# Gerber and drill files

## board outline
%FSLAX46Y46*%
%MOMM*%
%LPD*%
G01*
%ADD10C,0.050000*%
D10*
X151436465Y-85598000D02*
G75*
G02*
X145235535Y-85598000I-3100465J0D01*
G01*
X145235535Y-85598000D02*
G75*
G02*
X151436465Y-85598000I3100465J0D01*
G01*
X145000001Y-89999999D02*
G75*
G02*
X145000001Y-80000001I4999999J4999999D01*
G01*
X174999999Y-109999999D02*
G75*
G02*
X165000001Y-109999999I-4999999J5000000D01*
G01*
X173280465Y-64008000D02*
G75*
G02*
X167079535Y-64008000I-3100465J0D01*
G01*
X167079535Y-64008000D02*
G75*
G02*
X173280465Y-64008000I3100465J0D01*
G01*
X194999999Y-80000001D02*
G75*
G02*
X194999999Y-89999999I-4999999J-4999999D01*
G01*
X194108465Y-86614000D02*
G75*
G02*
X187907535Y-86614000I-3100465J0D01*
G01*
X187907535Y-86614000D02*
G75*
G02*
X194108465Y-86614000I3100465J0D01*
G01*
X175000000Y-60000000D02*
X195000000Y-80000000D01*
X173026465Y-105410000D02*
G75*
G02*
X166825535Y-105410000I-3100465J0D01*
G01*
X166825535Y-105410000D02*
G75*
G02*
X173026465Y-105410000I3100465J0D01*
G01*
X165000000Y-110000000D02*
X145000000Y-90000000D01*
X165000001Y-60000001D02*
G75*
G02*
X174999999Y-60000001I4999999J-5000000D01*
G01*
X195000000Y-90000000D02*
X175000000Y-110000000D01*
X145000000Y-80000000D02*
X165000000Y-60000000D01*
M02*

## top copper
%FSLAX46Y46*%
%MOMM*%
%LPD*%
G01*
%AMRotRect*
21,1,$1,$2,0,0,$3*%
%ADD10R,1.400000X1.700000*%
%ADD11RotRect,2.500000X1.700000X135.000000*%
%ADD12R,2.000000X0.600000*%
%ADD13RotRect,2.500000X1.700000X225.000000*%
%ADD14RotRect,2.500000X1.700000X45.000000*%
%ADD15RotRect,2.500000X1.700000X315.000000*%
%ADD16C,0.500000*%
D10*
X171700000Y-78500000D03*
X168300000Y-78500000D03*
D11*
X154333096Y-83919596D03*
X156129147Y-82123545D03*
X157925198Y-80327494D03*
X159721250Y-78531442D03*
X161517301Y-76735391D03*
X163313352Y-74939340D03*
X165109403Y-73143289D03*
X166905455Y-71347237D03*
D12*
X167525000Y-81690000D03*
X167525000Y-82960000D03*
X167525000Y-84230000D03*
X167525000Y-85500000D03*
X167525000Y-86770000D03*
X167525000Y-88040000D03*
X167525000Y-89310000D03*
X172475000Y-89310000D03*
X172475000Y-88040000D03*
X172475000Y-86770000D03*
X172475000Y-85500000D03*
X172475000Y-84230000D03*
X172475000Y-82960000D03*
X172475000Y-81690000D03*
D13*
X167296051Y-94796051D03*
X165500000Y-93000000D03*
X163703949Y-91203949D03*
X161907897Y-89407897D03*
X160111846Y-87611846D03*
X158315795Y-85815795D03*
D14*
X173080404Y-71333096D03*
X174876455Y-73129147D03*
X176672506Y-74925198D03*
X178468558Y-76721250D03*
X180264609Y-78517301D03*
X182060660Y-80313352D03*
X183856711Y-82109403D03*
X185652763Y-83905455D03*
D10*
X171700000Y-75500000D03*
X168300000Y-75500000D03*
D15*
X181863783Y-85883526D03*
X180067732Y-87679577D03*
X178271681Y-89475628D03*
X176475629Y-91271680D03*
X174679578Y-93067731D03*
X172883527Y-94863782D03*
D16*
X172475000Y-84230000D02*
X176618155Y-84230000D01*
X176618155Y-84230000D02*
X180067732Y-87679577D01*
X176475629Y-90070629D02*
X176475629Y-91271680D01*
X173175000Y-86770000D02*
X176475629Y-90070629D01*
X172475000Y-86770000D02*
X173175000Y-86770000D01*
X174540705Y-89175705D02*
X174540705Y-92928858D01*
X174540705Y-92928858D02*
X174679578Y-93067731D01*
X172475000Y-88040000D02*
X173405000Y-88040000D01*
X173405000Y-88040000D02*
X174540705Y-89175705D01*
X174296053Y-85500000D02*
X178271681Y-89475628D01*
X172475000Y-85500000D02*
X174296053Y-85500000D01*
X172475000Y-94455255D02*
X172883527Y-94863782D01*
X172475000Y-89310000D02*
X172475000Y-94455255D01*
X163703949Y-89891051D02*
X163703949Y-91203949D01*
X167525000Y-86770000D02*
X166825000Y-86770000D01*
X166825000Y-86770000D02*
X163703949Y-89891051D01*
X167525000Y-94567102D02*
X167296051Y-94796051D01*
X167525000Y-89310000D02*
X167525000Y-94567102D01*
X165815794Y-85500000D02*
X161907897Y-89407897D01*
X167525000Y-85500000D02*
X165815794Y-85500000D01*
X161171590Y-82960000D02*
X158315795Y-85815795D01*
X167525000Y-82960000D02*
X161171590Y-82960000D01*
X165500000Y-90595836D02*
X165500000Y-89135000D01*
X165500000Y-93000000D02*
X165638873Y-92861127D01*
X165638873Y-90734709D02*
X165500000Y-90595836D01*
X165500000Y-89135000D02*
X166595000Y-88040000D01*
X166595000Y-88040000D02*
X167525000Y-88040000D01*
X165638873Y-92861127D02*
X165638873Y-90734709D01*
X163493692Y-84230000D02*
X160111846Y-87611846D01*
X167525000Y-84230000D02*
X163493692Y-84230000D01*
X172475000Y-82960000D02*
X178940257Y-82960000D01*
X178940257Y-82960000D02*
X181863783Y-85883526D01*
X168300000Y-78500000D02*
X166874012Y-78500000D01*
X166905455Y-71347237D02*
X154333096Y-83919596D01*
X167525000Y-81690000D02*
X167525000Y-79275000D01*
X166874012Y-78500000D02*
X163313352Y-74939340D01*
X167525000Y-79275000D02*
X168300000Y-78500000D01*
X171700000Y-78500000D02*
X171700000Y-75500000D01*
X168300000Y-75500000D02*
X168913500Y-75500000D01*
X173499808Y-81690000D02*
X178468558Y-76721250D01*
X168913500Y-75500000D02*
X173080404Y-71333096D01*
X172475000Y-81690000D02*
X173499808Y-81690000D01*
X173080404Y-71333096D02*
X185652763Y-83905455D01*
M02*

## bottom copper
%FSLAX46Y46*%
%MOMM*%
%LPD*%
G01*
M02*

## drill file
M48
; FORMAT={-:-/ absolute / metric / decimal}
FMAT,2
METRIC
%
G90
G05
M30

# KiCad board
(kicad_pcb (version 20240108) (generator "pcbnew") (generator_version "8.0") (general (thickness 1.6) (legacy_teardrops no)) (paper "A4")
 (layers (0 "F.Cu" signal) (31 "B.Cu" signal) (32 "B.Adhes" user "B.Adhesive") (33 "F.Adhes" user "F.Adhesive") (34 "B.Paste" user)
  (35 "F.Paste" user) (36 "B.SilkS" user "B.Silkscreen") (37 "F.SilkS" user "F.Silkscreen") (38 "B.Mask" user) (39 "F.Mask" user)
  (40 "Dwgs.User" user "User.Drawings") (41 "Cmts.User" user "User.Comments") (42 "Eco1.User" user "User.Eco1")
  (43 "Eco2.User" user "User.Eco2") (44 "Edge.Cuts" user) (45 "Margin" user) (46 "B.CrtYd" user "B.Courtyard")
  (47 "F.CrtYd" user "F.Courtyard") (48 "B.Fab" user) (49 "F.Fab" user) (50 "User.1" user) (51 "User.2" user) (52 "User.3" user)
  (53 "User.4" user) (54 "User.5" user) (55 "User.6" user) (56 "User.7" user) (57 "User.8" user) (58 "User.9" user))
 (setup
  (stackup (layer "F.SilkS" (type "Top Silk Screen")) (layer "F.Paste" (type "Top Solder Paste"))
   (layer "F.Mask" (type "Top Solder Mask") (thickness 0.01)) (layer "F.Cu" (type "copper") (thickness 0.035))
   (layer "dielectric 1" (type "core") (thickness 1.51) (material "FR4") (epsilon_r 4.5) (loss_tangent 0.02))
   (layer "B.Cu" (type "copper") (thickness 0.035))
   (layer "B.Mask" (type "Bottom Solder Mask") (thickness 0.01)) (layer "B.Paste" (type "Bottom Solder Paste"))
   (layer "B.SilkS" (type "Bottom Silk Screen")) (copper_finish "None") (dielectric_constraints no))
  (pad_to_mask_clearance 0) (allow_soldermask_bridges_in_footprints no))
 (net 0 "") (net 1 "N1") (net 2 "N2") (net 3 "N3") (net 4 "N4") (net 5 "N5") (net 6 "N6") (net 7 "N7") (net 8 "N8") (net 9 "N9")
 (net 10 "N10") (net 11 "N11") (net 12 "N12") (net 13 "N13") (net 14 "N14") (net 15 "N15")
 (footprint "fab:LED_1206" (layer "F.Cu") (at 170 78.5 180)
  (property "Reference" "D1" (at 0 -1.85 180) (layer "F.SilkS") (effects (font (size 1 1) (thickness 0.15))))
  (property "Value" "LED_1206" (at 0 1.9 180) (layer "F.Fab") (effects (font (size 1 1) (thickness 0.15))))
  (pad "1" smd rect (at -1.7 0 180) (size 1.4 1.7) (layers "F.Cu" "F.Paste" "F.Mask") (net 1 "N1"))
  (pad "2" smd rect (at 1.7 0 180) (size 1.4 1.7) (layers "F.Cu" "F.Paste" "F.Mask") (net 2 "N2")))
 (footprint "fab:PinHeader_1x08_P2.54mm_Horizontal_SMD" (layer "F.Cu") (at 154.333096 83.919596 135)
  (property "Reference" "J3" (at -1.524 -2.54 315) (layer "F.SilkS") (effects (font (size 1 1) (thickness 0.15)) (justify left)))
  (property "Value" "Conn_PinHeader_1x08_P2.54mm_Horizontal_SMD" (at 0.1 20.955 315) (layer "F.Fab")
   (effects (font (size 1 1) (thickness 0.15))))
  (pad "1" smd rect (at 0 0 135) (size 2.5 1.7) (layers "F.Cu" "F.Paste" "F.Mask") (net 2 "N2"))
  (pad "2" smd rect (at 0 2.54 135) (size 2.5 1.7) (layers "F.Cu" "F.Paste" "F.Mask") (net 2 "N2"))
  (pad "3" smd rect (at 0 5.079999 135) (size 2.5 1.7) (layers "F.Cu" "F.Paste" "F.Mask") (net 2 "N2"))
  (pad "4" smd rect (at 0 7.62 135) (size 2.5 1.7) (layers "F.Cu" "F.Paste" "F.Mask") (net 2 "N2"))
  (pad "5" smd rect (at 0 10.16 135) (size 2.5 1.7) (layers "F.Cu" "F.Paste" "F.Mask") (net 2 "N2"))
  (pad "6" smd rect (at 0 12.7 135) (size 2.5 1.7) (layers "F.Cu" "F.Paste" "F.Mask") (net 2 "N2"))
  (pad "7" smd rect (at 0 15.24 135) (size 2.5 1.7) (layers "F.Cu" "F.Paste" "F.Mask") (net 2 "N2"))
  (pad "8" smd rect (at 0 17.780001 135) (size 2.5 1.7) (layers "F.Cu" "F.Paste" "F.Mask") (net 2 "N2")))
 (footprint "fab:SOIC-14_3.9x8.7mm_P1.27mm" (layer "F.Cu") (at 170 85.5)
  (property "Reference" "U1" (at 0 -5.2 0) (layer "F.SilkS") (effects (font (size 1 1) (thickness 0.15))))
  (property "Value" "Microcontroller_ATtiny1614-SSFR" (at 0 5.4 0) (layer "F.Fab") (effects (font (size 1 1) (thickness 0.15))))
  (pad "1" smd rect (at -2.475 -3.81) (size 2 0.6) (layers "F.Cu" "F.Paste" "F.Mask") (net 2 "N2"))
  (pad "2" smd rect (at -2.475 -2.54) (size 2 0.6) (layers "F.Cu" "F.Paste" "F.Mask") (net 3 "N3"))
  (pad "3" smd rect (at -2.475 -1.27) (size 2 0.6) (layers "F.Cu" "F.Paste" "F.Mask") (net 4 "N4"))
  (pad "4" smd rect (at -2.475 0) (size 2 0.6) (layers "F.Cu" "F.Paste" "F.Mask") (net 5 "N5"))
  (pad "5" smd rect (at -2.475 1.27) (size 2 0.6) (layers "F.Cu" "F.Paste" "F.Mask") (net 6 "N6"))
  (pad "6" smd rect (at -2.475 2.54) (size 2 0.6) (layers "F.Cu" "F.Paste" "F.Mask") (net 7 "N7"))
  (pad "7" smd rect (at -2.475 3.81) (size 2 0.6) (layers "F.Cu" "F.Paste" "F.Mask") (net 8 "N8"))
  (pad "8" smd rect (at 2.475 3.81) (size 2 0.6) (layers "F.Cu" "F.Paste" "F.Mask") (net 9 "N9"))
  (pad "9" smd rect (at 2.475 2.54) (size 2 0.6) (layers "F.Cu" "F.Paste" "F.Mask") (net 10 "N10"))
  (pad "10" smd rect (at 2.475 1.27) (size 2 0.6) (layers "F.Cu" "F.Paste" "F.Mask") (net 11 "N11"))
  (pad "11" smd rect (at 2.475 0) (size 2 0.6) (layers "F.Cu" "F.Paste" "F.Mask") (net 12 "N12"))
  (pad "12" smd rect (at 2.475 -1.27) (size 2 0.6) (layers "F.Cu" "F.Paste" "F.Mask") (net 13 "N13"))
  (pad "13" smd rect (at 2.475 -2.54) (size 2 0.6) (layers "F.Cu" "F.Paste" "F.Mask") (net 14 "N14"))
  (pad "14" smd rect (at 2.475 -3.81) (size 2 0.6) (layers "F.Cu" "F.Paste" "F.Mask") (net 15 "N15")))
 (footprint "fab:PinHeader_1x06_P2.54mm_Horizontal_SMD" (layer "F.Cu") (at 167.296051 94.796051 -135)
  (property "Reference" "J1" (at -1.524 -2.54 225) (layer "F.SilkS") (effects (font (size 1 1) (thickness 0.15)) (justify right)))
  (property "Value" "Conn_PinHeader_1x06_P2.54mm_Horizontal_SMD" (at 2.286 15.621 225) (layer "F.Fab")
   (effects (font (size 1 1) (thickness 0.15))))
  (pad "1" smd rect (at 0 0 225) (size 2.5 1.7) (layers "F.Cu" "F.Paste" "F.Mask") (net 8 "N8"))
  (pad "2" smd rect (at 0 2.54 225) (size 2.5 1.7) (layers "F.Cu" "F.Paste" "F.Mask") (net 7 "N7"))
  (pad "3" smd rect (at 0 5.079999 225) (size 2.5 1.7) (layers "F.Cu" "F.Paste" "F.Mask") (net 6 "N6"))
  (pad "4" smd rect (at 0 7.62 225) (size 2.5 1.7) (layers "F.Cu" "F.Paste" "F.Mask") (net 5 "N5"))
  (pad "5" smd rect (at 0 10.16 225) (size 2.5 1.7) (layers "F.Cu" "F.Paste" "F.Mask") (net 4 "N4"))
  (pad "6" smd rect (at 0 12.7 225) (size 2.5 1.7) (layers "F.Cu" "F.Paste" "F.Mask") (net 3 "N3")))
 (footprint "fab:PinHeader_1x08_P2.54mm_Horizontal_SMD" (layer "F.Cu") (at 173.080404 71.333096 45)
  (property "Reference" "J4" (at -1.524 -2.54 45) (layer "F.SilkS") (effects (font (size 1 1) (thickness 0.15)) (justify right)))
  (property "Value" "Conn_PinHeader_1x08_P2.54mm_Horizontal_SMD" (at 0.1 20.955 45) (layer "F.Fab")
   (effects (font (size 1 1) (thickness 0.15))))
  (pad "1" smd rect (at 0 0 45) (size 2.5 1.7) (layers "F.Cu" "F.Paste" "F.Mask") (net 15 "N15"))
  (pad "2" smd rect (at 0 2.54 45) (size 2.5 1.7) (layers "F.Cu" "F.Paste" "F.Mask") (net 15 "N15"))
  (pad "3" smd rect (at 0 5.079999 45) (size 2.5 1.7) (layers "F.Cu" "F.Paste" "F.Mask") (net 15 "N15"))
  (pad "4" smd rect (at 0 7.62 45) (size 2.5 1.7) (layers "F.Cu" "F.Paste" "F.Mask") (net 15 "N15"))
  (pad "5" smd rect (at 0 10.16 45) (size 2.5 1.7) (layers "F.Cu" "F.Paste" "F.Mask") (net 15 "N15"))
  (pad "6" smd rect (at 0 12.7 45) (size 2.5 1.7) (layers "F.Cu" "F.Paste" "F.Mask") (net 15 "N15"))
  (pad "7" smd rect (at 0 15.24 45) (size 2.5 1.7) (layers "F.Cu" "F.Paste" "F.Mask") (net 15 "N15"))
  (pad "8" smd rect (at 0 17.780001 45) (size 2.5 1.7) (layers "F.Cu" "F.Paste" "F.Mask") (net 15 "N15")))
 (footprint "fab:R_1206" (layer "F.Cu") (at 170 75.5 180)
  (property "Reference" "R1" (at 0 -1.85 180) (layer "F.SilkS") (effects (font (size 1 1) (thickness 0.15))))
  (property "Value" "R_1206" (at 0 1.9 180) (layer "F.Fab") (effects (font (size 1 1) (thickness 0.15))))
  (pad "1" smd rect (at -1.7 0 180) (size 1.4 1.7) (layers "F.Cu" "F.Paste" "F.Mask") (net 1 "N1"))
  (pad "2" smd rect (at 1.7 0 180) (size 1.4 1.7) (layers "F.Cu" "F.Paste" "F.Mask") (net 15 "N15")))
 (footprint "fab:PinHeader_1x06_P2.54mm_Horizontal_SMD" (layer "F.Cu") (at 181.863783 85.883526 -45)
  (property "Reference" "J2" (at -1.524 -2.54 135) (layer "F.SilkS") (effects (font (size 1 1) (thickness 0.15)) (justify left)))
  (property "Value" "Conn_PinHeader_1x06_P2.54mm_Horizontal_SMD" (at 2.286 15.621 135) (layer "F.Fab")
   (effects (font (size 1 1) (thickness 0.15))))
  (pad "1" smd rect (at 0 0 315) (size 2.5 1.7) (layers "F.Cu" "F.Paste" "F.Mask") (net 14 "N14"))
  (pad "2" smd rect (at 0 2.54 315) (size 2.5 1.7) (layers "F.Cu" "F.Paste" "F.Mask") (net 13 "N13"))
  (pad "3" smd rect (at 0 5.079999 315) (size 2.5 1.7) (layers "F.Cu" "F.Paste" "F.Mask") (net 12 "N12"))
  (pad "4" smd rect (at 0 7.62 315) (size 2.5 1.7) (layers "F.Cu" "F.Paste" "F.Mask") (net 11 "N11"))
  (pad "5" smd rect (at 0 10.16 315) (size 2.5 1.7) (layers "F.Cu" "F.Paste" "F.Mask") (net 10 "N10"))
  (pad "6" smd rect (at 0 12.7 315) (size 2.5 1.7) (layers "F.Cu" "F.Paste" "F.Mask") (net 9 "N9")))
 (gr_circle (center 148.336 85.598) (end 146.558 83.058) (stroke (width 0.05) (type default)) (fill none) (layer "Edge.Cuts"))
 (gr_arc (start 145.000001 89.999999) (mid 142.928934 85) (end 145.000001 80.000001) (stroke (width 0.05) (type default))
  (layer "Edge.Cuts"))
 (gr_arc (start 174.999999 109.999999) (mid 170 112.071066) (end 165.000001 109.999999) (stroke (width 0.05) (type default))
  (layer "Edge.Cuts"))
 (gr_circle (center 170.18 64.008) (end 168.402 61.468) (stroke (width 0.05) (type default)) (fill none) (layer "Edge.Cuts"))
 (gr_arc (start 194.999999 80.000001) (mid 197.071066 85) (end 194.999999 89.999999) (stroke (width 0.05) (type default))
  (layer "Edge.Cuts"))
 (gr_circle (center 191.008 86.614) (end 189.23 84.074) (stroke (width 0.05) (type default)) (fill none) (layer "Edge.Cuts"))
 (gr_line (start 175 60) (end 195 80) (stroke (width 0.05) (type default)) (layer "Edge.Cuts"))
 (gr_circle (center 169.926 105.41) (end 168.148 102.87) (stroke (width 0.05) (type default)) (fill none) (layer "Edge.Cuts"))
 (gr_line (start 165 110) (end 145 90) (stroke (width 0.05) (type default)) (layer "Edge.Cuts"))
 (gr_arc (start 165.000001 60.000001) (mid 170 57.928934) (end 174.999999 60.000001) (stroke (width 0.05) (type default))
  (layer "Edge.Cuts"))
 (gr_line (start 195 90) (end 175 110) (stroke (width 0.05) (type default)) (layer "Edge.Cuts"))
 (gr_line (start 145 80) (end 165 60) (stroke (width 0.05) (type default)) (layer "Edge.Cuts"))
 (segment (start 172.475 84.23) (end 176.618155 84.23) (width 0.5) (layer "F.Cu") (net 13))
 (segment (start 176.618155 84.23) (end 180.067732 87.679577) (width 0.5) (layer "F.Cu") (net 13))
 (segment (start 176.475629 90.070629) (end 176.475629 91.27168) (width 0.5) (layer "F.Cu") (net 11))
 (segment (start 173.175 86.77) (end 176.475629 90.070629) (width 0.5) (layer "F.Cu") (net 11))
 (segment (start 172.475 86.77) (end 173.175 86.77) (width 0.5) (layer "F.Cu") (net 11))
 (segment (start 174.540705 89.175705) (end 174.540705 92.928858) (width 0.5) (layer "F.Cu") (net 10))
 (segment (start 174.540705 92.928858) (end 174.679578 93.067731) (width 0.5) (layer "F.Cu") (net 10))
 (segment (start 172.475 88.04) (end 173.405 88.04) (width 0.5) (layer "F.Cu") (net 10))
 (segment (start 173.405 88.04) (end 174.540705 89.175705) (width 0.5) (layer "F.Cu") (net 10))
 (segment (start 174.296053 85.5) (end 178.271681 89.475628) (width 0.5) (layer "F.Cu") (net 12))
 (segment (start 172.475 85.5) (end 174.296053 85.5) (width 0.5) (layer "F.Cu") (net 12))
 (segment (start 172.475 94.455255) (end 172.883527 94.863782) (width 0.5) (layer "F.Cu") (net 9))
 (segment (start 172.475 89.31) (end 172.475 94.455255) (width 0.5) (layer "F.Cu") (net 9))
 (segment (start 163.703949 89.891051) (end 163.703949 91.203949) (width 0.5) (layer "F.Cu") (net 6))
 (segment (start 167.525 86.77) (end 166.825 86.77) (width 0.5) (layer "F.Cu") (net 6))
 (segment (start 166.825 86.77) (end 163.703949 89.891051) (width 0.5) (layer "F.Cu") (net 6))
 (segment (start 167.525 94.567102) (end 167.296051 94.796051) (width 0.5) (layer "F.Cu") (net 8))
 (segment (start 167.525 89.31) (end 167.525 94.567102) (width 0.5) (layer "F.Cu") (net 8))
 (segment (start 165.815794 85.5) (end 161.907897 89.407897) (width 0.5) (layer "F.Cu") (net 5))
 (segment (start 167.525 85.5) (end 165.815794 85.5) (width 0.5) (layer "F.Cu") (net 5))
 (segment (start 161.17159 82.96) (end 158.315795 85.815795) (width 0.5) (layer "F.Cu") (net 3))
 (segment (start 167.525 82.96) (end 161.17159 82.96) (width 0.5) (layer "F.Cu") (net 3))
 (segment (start 165.5 90.595836) (end 165.5 89.135) (width 0.5) (layer "F.Cu") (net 7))
 (segment (start 165.5 93) (end 165.638873 92.861127) (width 0.5) (layer "F.Cu") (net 7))
 (segment (start 165.638873 90.734709) (end 165.5 90.595836) (width 0.5) (layer "F.Cu") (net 7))
 (segment (start 165.5 89.135) (end 166.595 88.04) (width 0.5) (layer "F.Cu") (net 7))
 (segment (start 166.595 88.04) (end 167.525 88.04) (width 0.5) (layer "F.Cu") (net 7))
 (segment (start 165.638873 92.861127) (end 165.638873 90.734709) (width 0.5) (layer "F.Cu") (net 7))
 (segment (start 163.493692 84.23) (end 160.111846 87.611846) (width 0.5) (layer "F.Cu") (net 4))
 (segment (start 167.525 84.23) (end 163.493692 84.23) (width 0.5) (layer "F.Cu") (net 4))
 (segment (start 172.475 82.96) (end 178.940257 82.96) (width 0.5) (layer "F.Cu") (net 14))
 (segment (start 178.940257 82.96) (end 181.863783 85.883526) (width 0.5) (layer "F.Cu") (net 14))
 (segment (start 168.3 78.5) (end 166.874012 78.5) (width 0.5) (layer "F.Cu") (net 2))
 (segment (start 166.905455 71.347237) (end 154.333096 83.919596) (width 0.5) (layer "F.Cu") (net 2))
 (segment (start 167.525 81.69) (end 167.525 79.275) (width 0.5) (layer "F.Cu") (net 2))
 (segment (start 166.874012 78.5) (end 163.313352 74.93934) (width 0.5) (layer "F.Cu") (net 2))
 (segment (start 167.525 79.275) (end 168.3 78.5) (width 0.5) (layer "F.Cu") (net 2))
 (segment (start 171.7 78.5) (end 171.7 75.5) (width 0.5) (layer "F.Cu") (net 1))
 (segment (start 168.3 75.5) (end 168.9135 75.5) (width 0.5) (layer "F.Cu") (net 15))
 (segment (start 173.499808 81.69) (end 178.468558 76.72125) (width 0.5) (layer "F.Cu") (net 15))
 (segment (start 168.9135 75.5) (end 173.080404 71.333096) (width 0.5) (layer "F.Cu") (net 15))
 (segment (start 172.475 81.69) (end 173.499808 81.69) (width 0.5) (layer "F.Cu") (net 15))
 (segment (start 173.080404 71.333096) (end 185.652763 83.905455) (width 0.5) (layer "F.Cu") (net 15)))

